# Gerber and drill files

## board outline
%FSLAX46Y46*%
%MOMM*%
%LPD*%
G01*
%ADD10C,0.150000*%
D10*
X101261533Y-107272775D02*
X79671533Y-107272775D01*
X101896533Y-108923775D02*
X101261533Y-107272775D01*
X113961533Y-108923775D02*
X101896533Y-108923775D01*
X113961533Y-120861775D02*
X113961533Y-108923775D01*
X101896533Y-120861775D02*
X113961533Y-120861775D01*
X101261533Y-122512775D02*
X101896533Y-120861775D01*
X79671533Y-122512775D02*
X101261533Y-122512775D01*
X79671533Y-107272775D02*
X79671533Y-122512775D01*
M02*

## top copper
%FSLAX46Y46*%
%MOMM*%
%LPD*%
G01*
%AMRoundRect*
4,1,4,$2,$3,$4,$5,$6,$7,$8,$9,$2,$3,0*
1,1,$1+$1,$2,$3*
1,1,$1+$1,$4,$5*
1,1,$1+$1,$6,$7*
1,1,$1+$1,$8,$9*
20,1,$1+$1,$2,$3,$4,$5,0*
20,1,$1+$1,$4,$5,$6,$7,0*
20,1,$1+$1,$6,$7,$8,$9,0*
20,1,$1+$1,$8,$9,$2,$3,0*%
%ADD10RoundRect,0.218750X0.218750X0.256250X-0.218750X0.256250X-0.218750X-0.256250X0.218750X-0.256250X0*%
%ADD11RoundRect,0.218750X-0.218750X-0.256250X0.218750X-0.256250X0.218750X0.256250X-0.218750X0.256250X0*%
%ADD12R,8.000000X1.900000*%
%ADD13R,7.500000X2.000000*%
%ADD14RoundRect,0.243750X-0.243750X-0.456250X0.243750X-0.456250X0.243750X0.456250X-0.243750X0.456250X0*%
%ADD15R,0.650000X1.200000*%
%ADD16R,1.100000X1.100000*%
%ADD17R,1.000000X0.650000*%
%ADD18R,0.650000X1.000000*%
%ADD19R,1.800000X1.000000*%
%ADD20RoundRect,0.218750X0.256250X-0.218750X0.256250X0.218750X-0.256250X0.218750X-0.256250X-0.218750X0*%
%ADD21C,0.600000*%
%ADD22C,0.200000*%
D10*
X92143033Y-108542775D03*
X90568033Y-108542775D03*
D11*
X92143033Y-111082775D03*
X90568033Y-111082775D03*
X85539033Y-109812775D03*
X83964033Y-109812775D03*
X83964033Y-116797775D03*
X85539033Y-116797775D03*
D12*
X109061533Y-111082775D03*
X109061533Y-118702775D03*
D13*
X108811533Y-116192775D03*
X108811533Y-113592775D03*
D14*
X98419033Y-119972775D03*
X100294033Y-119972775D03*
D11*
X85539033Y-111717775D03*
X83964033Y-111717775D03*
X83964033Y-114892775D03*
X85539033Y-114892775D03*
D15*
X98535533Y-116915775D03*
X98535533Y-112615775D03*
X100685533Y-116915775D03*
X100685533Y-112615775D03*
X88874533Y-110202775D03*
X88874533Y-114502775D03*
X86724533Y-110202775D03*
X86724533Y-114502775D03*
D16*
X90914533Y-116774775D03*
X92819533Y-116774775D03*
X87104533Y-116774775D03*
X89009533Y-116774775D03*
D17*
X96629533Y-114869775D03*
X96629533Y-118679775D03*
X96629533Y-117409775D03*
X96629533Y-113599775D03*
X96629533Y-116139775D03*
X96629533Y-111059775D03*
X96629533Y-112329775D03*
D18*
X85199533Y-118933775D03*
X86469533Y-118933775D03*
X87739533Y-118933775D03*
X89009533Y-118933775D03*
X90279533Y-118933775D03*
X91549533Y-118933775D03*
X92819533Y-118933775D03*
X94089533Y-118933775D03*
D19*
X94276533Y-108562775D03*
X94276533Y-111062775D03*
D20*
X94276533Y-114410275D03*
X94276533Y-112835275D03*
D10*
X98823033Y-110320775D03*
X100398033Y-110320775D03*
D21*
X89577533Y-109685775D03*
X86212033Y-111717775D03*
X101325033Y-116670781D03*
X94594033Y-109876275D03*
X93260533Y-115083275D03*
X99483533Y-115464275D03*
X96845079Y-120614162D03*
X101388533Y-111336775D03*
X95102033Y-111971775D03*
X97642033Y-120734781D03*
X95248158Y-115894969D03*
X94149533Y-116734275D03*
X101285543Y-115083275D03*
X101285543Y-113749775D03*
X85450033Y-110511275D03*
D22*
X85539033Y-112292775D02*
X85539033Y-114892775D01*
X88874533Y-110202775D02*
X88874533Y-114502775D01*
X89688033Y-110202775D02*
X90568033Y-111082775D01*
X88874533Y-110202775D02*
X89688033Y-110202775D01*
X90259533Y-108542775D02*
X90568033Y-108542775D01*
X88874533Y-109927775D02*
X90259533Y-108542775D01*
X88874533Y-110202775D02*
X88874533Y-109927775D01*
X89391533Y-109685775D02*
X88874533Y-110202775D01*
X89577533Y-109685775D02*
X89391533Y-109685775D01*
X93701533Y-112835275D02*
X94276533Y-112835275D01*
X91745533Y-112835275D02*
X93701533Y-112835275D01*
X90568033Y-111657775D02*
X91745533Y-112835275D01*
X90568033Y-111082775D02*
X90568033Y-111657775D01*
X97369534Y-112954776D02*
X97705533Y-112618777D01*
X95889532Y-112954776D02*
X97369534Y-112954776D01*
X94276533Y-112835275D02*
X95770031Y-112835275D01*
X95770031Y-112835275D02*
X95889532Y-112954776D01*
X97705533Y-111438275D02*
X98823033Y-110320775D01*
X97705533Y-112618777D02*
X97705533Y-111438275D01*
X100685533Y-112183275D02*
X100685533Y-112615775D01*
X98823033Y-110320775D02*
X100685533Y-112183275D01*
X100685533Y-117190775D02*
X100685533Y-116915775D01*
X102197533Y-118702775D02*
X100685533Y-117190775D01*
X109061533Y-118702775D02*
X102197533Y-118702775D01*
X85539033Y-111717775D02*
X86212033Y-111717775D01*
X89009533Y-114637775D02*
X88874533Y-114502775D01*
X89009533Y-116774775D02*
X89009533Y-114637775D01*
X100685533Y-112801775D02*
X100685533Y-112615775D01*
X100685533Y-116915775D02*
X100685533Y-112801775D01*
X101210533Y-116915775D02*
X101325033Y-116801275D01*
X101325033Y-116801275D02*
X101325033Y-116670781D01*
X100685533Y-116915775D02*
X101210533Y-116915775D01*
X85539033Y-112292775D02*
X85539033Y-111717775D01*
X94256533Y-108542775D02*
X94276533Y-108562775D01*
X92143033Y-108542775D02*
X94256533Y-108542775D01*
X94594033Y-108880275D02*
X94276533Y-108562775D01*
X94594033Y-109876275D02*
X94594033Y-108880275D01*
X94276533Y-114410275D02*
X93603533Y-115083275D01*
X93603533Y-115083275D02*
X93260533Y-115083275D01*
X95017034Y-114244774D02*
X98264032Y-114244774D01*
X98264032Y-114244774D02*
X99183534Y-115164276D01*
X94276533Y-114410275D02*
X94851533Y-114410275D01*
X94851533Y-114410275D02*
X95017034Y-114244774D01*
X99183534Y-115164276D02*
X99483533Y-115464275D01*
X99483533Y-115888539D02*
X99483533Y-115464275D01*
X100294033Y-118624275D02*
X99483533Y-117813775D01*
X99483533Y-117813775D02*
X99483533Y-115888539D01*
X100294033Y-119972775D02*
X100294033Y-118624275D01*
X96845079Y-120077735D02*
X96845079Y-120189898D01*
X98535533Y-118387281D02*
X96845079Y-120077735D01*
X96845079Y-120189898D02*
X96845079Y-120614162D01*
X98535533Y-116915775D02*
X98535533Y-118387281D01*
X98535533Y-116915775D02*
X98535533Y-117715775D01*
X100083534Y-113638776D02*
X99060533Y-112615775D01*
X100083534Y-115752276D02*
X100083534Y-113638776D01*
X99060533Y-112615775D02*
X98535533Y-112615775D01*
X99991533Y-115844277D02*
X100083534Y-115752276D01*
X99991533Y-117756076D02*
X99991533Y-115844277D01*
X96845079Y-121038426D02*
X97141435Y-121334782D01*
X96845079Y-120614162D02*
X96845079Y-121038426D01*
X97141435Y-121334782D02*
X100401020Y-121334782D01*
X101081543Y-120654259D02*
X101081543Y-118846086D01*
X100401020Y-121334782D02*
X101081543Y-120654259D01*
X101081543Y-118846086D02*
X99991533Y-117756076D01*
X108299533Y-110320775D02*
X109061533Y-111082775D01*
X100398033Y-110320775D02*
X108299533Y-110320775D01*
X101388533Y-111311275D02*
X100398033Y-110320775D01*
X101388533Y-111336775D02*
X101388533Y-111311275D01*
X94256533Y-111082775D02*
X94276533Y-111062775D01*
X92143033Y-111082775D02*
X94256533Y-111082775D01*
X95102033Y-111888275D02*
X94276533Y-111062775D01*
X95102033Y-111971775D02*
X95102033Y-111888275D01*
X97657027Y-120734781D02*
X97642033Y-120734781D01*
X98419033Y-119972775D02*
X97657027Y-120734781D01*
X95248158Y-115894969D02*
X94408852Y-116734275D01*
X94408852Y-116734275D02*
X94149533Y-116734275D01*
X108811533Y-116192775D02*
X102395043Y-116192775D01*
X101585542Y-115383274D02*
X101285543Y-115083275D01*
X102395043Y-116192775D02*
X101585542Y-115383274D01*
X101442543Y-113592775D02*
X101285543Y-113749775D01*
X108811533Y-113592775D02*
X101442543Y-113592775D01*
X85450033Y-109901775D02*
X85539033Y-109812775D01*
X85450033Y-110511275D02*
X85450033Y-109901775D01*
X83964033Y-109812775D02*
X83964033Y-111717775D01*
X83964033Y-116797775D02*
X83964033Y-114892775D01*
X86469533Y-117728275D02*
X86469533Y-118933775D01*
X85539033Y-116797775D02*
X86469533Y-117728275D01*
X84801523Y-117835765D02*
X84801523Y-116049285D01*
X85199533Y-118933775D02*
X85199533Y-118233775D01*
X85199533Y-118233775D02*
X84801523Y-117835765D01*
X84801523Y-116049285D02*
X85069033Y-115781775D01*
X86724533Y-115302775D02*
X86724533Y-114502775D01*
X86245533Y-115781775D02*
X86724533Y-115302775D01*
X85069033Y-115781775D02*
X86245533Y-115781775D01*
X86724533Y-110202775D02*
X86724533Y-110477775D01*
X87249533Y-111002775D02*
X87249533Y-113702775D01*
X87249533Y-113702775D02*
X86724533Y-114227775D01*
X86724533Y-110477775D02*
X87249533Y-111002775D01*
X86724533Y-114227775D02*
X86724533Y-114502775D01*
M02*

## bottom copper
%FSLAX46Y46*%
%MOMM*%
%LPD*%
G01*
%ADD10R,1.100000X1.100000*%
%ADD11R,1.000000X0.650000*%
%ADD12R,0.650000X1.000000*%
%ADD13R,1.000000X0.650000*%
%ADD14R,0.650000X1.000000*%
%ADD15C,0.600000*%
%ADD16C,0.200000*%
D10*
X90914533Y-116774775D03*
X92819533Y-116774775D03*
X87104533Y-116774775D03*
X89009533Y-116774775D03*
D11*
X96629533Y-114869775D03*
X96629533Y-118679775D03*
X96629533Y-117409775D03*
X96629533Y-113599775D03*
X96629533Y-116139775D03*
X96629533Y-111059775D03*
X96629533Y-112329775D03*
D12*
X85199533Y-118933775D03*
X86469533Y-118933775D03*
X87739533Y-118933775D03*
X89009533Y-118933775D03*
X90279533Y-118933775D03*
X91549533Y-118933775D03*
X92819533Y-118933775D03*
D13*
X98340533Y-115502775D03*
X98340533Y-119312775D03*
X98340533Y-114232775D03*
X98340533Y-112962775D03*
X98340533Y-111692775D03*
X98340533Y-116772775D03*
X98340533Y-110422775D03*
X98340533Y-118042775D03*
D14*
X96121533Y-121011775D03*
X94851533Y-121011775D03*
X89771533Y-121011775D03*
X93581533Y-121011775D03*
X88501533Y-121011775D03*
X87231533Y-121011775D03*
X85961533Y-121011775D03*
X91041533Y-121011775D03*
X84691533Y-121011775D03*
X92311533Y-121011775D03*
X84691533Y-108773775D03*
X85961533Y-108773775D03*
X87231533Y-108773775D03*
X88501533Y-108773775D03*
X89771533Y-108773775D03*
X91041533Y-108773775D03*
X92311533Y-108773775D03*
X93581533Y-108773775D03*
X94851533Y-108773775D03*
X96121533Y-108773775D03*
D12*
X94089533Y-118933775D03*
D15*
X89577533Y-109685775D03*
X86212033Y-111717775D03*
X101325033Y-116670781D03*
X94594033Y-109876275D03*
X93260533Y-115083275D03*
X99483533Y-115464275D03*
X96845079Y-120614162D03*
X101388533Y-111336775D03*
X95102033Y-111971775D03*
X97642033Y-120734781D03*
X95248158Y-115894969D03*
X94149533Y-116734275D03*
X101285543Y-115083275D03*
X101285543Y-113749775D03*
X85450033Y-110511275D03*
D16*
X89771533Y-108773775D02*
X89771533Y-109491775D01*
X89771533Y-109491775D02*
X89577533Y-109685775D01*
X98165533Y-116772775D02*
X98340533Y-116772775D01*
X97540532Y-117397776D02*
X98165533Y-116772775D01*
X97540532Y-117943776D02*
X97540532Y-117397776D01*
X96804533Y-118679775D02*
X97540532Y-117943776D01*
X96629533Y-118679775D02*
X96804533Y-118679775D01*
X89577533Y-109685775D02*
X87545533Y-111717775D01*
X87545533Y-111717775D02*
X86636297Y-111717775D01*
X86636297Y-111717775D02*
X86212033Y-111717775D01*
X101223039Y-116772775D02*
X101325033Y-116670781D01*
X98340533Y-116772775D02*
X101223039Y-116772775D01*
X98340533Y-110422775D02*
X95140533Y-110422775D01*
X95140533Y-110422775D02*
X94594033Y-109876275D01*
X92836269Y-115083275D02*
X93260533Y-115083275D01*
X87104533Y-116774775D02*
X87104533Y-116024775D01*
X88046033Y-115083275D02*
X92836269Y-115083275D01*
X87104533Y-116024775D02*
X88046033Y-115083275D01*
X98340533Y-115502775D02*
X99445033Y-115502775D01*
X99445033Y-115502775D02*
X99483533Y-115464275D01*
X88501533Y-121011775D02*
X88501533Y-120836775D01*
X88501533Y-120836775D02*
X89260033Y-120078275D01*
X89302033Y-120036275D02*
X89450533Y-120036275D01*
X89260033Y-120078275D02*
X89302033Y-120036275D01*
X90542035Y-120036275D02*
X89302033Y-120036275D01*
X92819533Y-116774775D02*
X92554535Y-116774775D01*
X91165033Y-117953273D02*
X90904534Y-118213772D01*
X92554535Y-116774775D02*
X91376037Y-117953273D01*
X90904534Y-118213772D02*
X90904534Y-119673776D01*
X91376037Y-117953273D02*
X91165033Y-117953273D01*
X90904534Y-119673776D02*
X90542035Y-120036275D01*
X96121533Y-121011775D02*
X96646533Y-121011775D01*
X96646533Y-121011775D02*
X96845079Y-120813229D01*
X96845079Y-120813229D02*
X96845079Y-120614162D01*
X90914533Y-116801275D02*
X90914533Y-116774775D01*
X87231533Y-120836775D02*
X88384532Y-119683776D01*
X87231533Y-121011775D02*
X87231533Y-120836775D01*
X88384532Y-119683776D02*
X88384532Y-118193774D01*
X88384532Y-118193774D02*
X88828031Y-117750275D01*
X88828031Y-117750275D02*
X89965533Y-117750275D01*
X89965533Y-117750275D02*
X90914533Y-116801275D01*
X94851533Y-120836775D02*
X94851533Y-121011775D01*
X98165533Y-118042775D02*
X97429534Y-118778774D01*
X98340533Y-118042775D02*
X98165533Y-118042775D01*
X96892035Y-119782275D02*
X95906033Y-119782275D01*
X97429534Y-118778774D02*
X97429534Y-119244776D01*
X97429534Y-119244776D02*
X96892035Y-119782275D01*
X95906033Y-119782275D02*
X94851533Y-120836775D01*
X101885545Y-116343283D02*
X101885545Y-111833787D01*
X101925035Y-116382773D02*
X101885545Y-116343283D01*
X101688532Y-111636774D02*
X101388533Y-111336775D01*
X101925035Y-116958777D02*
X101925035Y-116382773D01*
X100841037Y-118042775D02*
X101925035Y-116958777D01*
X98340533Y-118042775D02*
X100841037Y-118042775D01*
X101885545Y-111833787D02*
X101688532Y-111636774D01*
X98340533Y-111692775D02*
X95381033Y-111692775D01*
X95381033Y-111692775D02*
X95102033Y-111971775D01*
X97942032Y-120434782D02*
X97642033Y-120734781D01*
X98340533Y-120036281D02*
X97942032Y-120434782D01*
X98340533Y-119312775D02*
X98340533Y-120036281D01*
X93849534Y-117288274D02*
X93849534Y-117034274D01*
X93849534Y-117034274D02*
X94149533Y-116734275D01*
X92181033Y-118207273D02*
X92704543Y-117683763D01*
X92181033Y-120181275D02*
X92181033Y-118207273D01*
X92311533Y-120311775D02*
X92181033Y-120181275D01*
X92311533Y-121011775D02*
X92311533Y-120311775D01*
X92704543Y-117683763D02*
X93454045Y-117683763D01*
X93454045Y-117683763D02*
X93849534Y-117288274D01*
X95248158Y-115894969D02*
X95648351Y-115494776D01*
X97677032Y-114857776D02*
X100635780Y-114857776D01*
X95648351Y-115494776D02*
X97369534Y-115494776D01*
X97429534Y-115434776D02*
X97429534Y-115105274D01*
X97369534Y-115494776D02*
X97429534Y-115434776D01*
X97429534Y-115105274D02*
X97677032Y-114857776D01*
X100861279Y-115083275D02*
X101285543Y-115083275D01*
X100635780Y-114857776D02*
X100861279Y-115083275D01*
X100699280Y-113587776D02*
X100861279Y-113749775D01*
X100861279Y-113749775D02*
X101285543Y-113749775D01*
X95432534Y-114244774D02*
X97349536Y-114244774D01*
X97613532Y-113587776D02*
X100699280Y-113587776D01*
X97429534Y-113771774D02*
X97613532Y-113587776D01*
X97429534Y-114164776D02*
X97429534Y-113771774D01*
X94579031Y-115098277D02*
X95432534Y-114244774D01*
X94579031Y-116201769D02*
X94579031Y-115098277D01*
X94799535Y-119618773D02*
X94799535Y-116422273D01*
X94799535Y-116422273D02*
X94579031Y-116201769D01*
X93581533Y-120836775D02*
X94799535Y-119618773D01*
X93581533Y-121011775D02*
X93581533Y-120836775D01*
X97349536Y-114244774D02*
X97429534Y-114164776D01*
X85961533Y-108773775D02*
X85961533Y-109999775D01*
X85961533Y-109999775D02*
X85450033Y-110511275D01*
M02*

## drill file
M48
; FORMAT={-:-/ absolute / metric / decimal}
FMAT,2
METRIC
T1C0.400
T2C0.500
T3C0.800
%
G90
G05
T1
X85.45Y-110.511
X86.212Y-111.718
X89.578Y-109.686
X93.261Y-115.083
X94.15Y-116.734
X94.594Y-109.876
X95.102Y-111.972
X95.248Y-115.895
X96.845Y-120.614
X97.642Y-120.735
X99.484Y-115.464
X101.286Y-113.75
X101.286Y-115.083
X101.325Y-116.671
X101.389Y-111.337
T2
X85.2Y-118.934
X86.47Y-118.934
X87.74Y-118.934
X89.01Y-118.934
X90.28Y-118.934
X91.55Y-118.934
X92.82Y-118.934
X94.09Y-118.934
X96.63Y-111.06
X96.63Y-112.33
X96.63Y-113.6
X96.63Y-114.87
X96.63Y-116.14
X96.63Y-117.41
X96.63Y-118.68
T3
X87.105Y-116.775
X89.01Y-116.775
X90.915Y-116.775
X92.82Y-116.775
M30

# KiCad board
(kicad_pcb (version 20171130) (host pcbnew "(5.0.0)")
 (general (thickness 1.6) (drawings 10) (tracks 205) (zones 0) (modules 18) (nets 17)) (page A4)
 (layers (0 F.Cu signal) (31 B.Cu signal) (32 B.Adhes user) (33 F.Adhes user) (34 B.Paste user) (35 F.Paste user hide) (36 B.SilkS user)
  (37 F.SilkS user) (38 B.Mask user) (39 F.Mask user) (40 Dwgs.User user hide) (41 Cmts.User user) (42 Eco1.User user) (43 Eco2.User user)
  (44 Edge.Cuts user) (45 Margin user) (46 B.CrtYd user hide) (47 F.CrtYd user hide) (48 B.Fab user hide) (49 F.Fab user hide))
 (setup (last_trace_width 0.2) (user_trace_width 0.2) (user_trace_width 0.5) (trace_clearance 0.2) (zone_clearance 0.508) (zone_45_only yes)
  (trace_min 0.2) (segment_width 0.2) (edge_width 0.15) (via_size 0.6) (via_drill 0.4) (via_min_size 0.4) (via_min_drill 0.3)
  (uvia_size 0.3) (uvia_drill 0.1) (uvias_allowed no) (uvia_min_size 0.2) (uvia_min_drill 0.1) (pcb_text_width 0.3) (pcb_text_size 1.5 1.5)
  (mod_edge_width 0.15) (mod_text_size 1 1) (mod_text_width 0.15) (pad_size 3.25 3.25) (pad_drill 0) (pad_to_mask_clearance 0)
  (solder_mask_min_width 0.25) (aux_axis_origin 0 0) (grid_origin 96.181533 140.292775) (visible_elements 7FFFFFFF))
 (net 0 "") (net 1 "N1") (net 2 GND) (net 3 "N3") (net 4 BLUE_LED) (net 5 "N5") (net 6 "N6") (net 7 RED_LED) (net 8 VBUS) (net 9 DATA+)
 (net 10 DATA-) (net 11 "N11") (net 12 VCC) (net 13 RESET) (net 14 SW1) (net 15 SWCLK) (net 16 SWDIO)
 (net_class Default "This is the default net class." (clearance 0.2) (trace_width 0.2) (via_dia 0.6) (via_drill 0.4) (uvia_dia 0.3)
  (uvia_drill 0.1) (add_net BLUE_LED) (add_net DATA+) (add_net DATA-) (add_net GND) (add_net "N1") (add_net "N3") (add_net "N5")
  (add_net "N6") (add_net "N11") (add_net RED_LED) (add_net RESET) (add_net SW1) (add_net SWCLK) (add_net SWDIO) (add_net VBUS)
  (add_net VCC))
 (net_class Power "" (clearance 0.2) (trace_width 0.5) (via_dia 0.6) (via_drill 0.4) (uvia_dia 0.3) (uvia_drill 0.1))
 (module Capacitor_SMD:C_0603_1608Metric (layer F.Cu) (at 91.355533 108.542775 180)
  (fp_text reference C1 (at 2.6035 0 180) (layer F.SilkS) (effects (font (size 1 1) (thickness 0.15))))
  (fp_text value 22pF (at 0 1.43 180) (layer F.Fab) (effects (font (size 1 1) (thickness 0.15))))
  (pad 1 smd roundrect (at -0.7875 0 180) (size 0.875 0.95) (layers F.Cu F.Paste F.Mask) (roundrect_rratio 0.25) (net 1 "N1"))
  (pad 2 smd roundrect (at 0.7875 0 180) (size 0.875 0.95) (layers F.Cu F.Paste F.Mask) (roundrect_rratio 0.25) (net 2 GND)))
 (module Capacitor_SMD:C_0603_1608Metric (layer F.Cu) (at 91.355533 111.082775)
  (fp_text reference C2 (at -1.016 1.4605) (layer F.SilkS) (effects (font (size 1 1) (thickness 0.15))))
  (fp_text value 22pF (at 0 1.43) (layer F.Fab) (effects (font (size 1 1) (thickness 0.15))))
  (pad 2 smd roundrect (at 0.7875 0) (size 0.875 0.95) (layers F.Cu F.Paste F.Mask) (roundrect_rratio 0.25) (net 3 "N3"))
  (pad 1 smd roundrect (at -0.7875 0) (size 0.875 0.95) (layers F.Cu F.Paste F.Mask) (roundrect_rratio 0.25) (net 2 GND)))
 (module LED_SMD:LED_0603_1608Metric (layer F.Cu) (at 84.751533 109.812775)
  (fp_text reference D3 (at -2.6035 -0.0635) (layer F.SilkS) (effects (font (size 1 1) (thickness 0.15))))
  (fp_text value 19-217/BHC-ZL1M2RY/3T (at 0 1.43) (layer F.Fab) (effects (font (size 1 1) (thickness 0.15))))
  (pad 2 smd roundrect (at 0.7875 0) (size 0.875 0.95) (layers F.Cu F.Paste F.Mask) (roundrect_rratio 0.25) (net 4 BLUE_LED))
  (pad 1 smd roundrect (at -0.7875 0) (size 0.875 0.95) (layers F.Cu F.Paste F.Mask) (roundrect_rratio 0.25) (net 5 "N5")))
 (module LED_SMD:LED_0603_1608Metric (layer F.Cu) (at 84.751533 116.797775)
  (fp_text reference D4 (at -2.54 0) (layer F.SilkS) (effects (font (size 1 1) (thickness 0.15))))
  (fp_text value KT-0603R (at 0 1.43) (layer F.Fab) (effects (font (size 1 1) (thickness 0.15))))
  (pad 1 smd roundrect (at -0.7875 0) (size 0.875 0.95) (layers F.Cu F.Paste F.Mask) (roundrect_rratio 0.25) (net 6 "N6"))
  (pad 2 smd roundrect (at 0.7875 0) (size 0.875 0.95) (layers F.Cu F.Paste F.Mask) (roundrect_rratio 0.25) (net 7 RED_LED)))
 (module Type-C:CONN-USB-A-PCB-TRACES (layer F.Cu) (at 113.961533 114.892775 90)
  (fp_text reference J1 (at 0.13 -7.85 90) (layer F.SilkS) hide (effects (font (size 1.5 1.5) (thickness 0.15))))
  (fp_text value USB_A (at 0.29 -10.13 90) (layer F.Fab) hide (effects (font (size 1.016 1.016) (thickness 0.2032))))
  (pad 1 connect rect (at 3.81 -4.9 90) (size 1.9 8) (layers F.Cu F.Mask) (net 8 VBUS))
  (pad 4 connect rect (at -3.81 -4.9 90) (size 1.9 8) (layers F.Cu F.Mask) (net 2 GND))
  (pad 3 connect rect (at -1.3 -5.15 90) (size 2 7.5) (layers F.Cu F.Mask) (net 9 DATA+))
  (pad 2 connect rect (at 1.3 -5.15 90) (size 2 7.5) (layers F.Cu F.Mask) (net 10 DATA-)))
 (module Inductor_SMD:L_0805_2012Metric (layer F.Cu) (at 99.356533 119.972775)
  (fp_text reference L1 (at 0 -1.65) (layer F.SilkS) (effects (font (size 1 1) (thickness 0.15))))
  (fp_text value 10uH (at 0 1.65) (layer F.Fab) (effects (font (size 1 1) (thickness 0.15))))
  (pad 1 smd roundrect (at -0.9375 0) (size 0.975 1.4) (layers F.Cu F.Paste F.Mask) (roundrect_rratio 0.25) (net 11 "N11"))
  (pad 2 smd roundrect (at 0.9375 0) (size 0.975 1.4) (layers F.Cu F.Paste F.Mask) (roundrect_rratio 0.25) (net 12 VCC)))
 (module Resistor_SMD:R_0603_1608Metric (layer F.Cu) (at 84.751533 111.717775)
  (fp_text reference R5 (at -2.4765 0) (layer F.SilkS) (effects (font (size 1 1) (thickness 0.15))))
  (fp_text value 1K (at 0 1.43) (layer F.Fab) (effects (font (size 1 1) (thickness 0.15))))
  (pad 2 smd roundrect (at 0.7875 0) (size 0.875 0.95) (layers F.Cu F.Paste F.Mask) (roundrect_rratio 0.25) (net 2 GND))
  (pad 1 smd roundrect (at -0.7875 0) (size 0.875 0.95) (layers F.Cu F.Paste F.Mask) (roundrect_rratio 0.25) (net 5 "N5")))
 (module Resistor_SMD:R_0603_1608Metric (layer F.Cu) (at 84.751533 114.892775)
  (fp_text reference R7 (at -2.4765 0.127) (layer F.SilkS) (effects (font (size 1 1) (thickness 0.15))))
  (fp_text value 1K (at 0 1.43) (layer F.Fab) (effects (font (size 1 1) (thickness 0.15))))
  (pad 1 smd roundrect (at -0.7875 0) (size 0.875 0.95) (layers F.Cu F.Paste F.Mask) (roundrect_rratio 0.25) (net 6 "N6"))
  (pad 2 smd roundrect (at 0.7875 0) (size 0.875 0.95) (layers F.Cu F.Paste F.Mask) (roundrect_rratio 0.25) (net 2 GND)))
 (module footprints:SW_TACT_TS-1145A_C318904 (layer F.Cu) (at 99.610533 114.765775 270)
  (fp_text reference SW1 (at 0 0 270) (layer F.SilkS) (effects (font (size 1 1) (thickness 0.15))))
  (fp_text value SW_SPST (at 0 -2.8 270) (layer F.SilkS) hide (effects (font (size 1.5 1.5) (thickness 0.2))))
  (pad 2 smd rect (at 2.15 1.075 270) (size 1.2 0.65) (layers F.Cu F.Paste F.Mask) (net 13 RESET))
  (pad 2 smd rect (at -2.15 1.075 270) (size 1.2 0.65) (layers F.Cu F.Paste F.Mask) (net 13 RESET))
  (pad 1 smd rect (at 2.15 -1.075 270) (size 1.2 0.65) (layers F.Cu F.Paste F.Mask) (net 2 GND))
  (pad 1 smd rect (at -2.15 -1.075 270) (size 1.2 0.65) (layers F.Cu F.Paste F.Mask) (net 2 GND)))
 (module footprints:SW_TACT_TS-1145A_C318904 (layer F.Cu) (at 87.799533 112.352775 270)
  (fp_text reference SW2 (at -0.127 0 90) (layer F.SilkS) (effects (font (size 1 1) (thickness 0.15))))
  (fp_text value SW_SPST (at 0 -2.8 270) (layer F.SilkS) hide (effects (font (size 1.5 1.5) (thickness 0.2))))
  (pad 1 smd rect (at -2.15 -1.075 270) (size 1.2 0.65) (layers F.Cu F.Paste F.Mask) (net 2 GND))
  (pad 1 smd rect (at 2.15 -1.075 270) (size 1.2 0.65) (layers F.Cu F.Paste F.Mask) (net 2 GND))
  (pad 2 smd rect (at -2.15 1.075 270) (size 1.2 0.65) (layers F.Cu F.Paste F.Mask) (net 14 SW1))
  (pad 2 smd rect (at 2.15 1.075 270) (size 1.2 0.65) (layers F.Cu F.Paste F.Mask) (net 14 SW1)))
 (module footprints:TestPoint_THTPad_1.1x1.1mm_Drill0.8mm (layer F.Cu) (at 90.914533 116.774775)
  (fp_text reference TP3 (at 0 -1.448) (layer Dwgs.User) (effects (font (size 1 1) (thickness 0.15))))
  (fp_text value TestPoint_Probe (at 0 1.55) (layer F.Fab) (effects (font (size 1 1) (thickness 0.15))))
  (pad 1 thru_hole rect (at 0 0) (size 1.1 1.1) (drill 0.8) (layers *.Cu *.Mask) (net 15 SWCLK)))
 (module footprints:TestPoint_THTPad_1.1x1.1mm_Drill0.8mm (layer F.Cu) (at 92.819533 116.774775)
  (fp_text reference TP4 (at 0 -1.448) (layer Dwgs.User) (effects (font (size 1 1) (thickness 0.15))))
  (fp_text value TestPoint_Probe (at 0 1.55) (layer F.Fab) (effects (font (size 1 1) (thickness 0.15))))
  (pad 1 thru_hole rect (at 0 0) (size 1.1 1.1) (drill 0.8) (layers *.Cu *.Mask) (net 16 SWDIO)))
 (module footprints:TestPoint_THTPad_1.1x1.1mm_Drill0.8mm (layer F.Cu) (at 87.104533 116.774775)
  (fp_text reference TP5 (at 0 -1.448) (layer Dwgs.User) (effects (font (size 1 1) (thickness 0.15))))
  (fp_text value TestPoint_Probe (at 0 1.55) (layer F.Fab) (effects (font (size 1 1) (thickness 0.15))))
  (pad 1 thru_hole rect (at 0 0) (size 1.1 1.1) (drill 0.8) (layers *.Cu *.Mask) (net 12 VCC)))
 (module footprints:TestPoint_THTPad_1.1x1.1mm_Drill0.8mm (layer F.Cu) (at 89.009533 116.774775)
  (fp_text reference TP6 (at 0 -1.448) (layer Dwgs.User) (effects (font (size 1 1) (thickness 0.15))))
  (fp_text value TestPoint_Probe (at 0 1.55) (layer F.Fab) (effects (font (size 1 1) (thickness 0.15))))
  (pad 1 thru_hole rect (at 0 0) (size 1.1 1.1) (drill 0.8) (layers *.Cu *.Mask) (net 2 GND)))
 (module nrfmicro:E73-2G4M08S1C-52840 (layer B.Cu) (at 98.721533 114.892775 180)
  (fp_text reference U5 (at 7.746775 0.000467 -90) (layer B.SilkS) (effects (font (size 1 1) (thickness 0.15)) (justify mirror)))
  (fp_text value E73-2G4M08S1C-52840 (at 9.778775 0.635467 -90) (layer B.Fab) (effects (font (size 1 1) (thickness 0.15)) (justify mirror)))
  (pad 18 thru_hole rect (at 2.092 0.023 90) (size 0.65 1) (drill 0.5) (layers *.Cu *.Mask))
  (pad 24 thru_hole rect (at 2.092 -3.787 90) (size 0.65 1) (drill 0.5) (layers *.Cu *.Mask) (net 2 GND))
  (pad 22 thru_hole rect (at 2.092 -2.517 90) (size 0.65 1) (drill 0.5) (layers *.Cu *.Mask))
  (pad 16 thru_hole rect (at 2.092 1.293 90) (size 0.65 1) (drill 0.5) (layers *.Cu *.Mask))
  (pad 20 thru_hole rect (at 2.092 -1.247 90) (size 0.65 1) (drill 0.5) (layers *.Cu *.Mask))
  (pad 12 thru_hole rect (at 2.092 3.833 90) (size 0.65 1) (drill 0.5) (layers *.Cu *.Mask))
  (pad 14 thru_hole rect (at 2.092 2.563 90) (size 0.65 1) (drill 0.5) (layers *.Cu *.Mask))
  (pad 42 thru_hole rect (at 13.522 -4.041 180) (size 0.65 1) (drill 0.5) (layers *.Cu *.Mask) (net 14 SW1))
  (pad 40 thru_hole rect (at 12.252 -4.041 180) (size 0.65 1) (drill 0.5) (layers *.Cu *.Mask) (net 7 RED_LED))
  (pad 38 thru_hole rect (at 10.982 -4.041 180) (size 0.65 1) (drill 0.5) (layers *.Cu *.Mask))
  (pad 36 thru_hole rect (at 9.712 -4.041 180) (size 0.65 1) (drill 0.5) (layers *.Cu *.Mask))
  (pad 34 thru_hole rect (at 8.442 -4.041 180) (size 0.65 1) (drill 0.5) (layers *.Cu *.Mask))
  (pad 32 thru_hole rect (at 7.172 -4.041 180) (size 0.65 1) (drill 0.5) (layers *.Cu *.Mask))
  (pad 30 thru_hole rect (at 5.902 -4.041 180) (size 0.65 1) (drill 0.5) (layers *.Cu *.Mask))
  (pad 19 smd rect (at 0.381 -0.61 90) (size 0.65 1) (layers B.Cu B.Paste B.Mask) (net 12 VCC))
  (pad 25 smd rect (at 0.381 -4.42 90) (size 0.65 1) (layers B.Cu B.Paste B.Mask) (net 11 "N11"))
  (pad 17 smd rect (at 0.381 0.66 90) (size 0.65 1) (layers B.Cu B.Paste B.Mask))
  (pad 15 smd rect (at 0.381 1.93 90) (size 0.65 1) (layers B.Cu B.Paste B.Mask))
  (pad 13 smd rect (at 0.381 3.2 90) (size 0.65 1) (layers B.Cu B.Paste B.Mask) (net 3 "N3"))
  (pad 21 smd rect (at 0.381 -1.88 90) (size 0.65 1) (layers B.Cu B.Paste B.Mask) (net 2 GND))
  (pad 11 smd rect (at 0.381 4.47 90) (size 0.65 1) (layers B.Cu B.Paste B.Mask) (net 1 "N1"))
  (pad 23 smd rect (at 0.381 -3.15 90) (size 0.65 1) (layers B.Cu B.Paste B.Mask) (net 8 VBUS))
  (pad 26 smd rect (at 2.6 -6.119 180) (size 0.65 1) (layers B.Cu B.Paste B.Mask) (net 13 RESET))
  (pad 27 smd rect (at 3.87 -6.119 180) (size 0.65 1) (layers B.Cu B.Paste B.Mask) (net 8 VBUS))
  (pad 35 smd rect (at 8.95 -6.119 180) (size 0.65 1) (layers B.Cu B.Paste B.Mask))
  (pad 29 smd rect (at 5.14 -6.119 180) (size 0.65 1) (layers B.Cu B.Paste B.Mask) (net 10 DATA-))
  (pad 37 smd rect (at 10.22 -6.119 180) (size 0.65 1) (layers B.Cu B.Paste B.Mask) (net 16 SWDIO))
  (pad 39 smd rect (at 11.49 -6.119 180) (size 0.65 1) (layers B.Cu B.Paste B.Mask) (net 15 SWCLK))
  (pad 41 smd rect (at 12.76 -6.119 180) (size 0.65 1) (layers B.Cu B.Paste B.Mask))
  (pad 33 smd rect (at 7.68 -6.119 180) (size 0.65 1) (layers B.Cu B.Paste B.Mask))
  (pad 43 smd rect (at 14.03 -6.119 180) (size 0.65 1) (layers B.Cu B.Paste B.Mask))
  (pad 31 smd rect (at 6.41 -6.119 180) (size 0.65 1) (layers B.Cu B.Paste B.Mask) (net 9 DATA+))
  (pad 1 smd rect (at 14.03 6.119 180) (size 0.65 1) (layers B.Cu B.Paste B.Mask))
  (pad 2 smd rect (at 12.76 6.119 180) (size 0.65 1) (layers B.Cu B.Paste B.Mask) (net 4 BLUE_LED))
  (pad 3 smd rect (at 11.49 6.119 180) (size 0.65 1) (layers B.Cu B.Paste B.Mask))
  (pad 4 smd rect (at 10.22 6.119 180) (size 0.65 1) (layers B.Cu B.Paste B.Mask))
  (pad 5 smd rect (at 8.95 6.119 180) (size 0.65 1) (layers B.Cu B.Paste B.Mask) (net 2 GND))
  (pad 6 smd rect (at 7.68 6.119 180) (size 0.65 1) (layers B.Cu B.Paste B.Mask))
  (pad 7 smd rect (at 6.41 6.119 180) (size 0.65 1) (layers B.Cu B.Paste B.Mask))
  (pad 8 smd rect (at 5.14 6.119 180) (size 0.65 1) (layers B.Cu B.Paste B.Mask))
  (pad 9 smd rect (at 3.87 6.119 180) (size 0.65 1) (layers B.Cu B.Paste B.Mask))
  (pad 10 smd rect (at 2.6 6.119 180) (size 0.65 1) (layers B.Cu B.Paste B.Mask))
  (pad 28 thru_hole rect (at 4.632 -4.041 180) (size 0.65 1) (drill 0.5) (layers *.Cu *.Mask)))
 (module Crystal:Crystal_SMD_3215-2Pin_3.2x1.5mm (layer F.Cu) (at 94.276533 109.812775 90)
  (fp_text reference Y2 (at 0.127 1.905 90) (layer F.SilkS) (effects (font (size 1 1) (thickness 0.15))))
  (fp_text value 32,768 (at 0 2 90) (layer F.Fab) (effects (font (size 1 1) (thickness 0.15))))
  (pad 1 smd rect (at 1.25 0 90) (size 1 1.8) (layers F.Cu F.Paste F.Mask) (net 1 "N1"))
  (pad 2 smd rect (at -1.25 0 90) (size 1 1.8) (layers F.Cu F.Paste F.Mask) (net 3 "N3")))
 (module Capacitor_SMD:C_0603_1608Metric (layer F.Cu) (at 94.276533 113.622775 90)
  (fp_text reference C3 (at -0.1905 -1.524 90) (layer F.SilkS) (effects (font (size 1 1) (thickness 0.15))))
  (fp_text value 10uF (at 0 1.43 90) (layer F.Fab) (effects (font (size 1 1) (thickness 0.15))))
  (pad 1 smd roundrect (at -0.7875 0 90) (size 0.875 0.95) (layers F.Cu F.Paste F.Mask) (roundrect_rratio 0.25) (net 12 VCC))
  (pad 2 smd roundrect (at 0.7875 0 90) (size 0.875 0.95) (layers F.Cu F.Paste F.Mask) (roundrect_rratio 0.25) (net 2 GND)))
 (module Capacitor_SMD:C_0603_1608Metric (layer F.Cu) (at 99.610533 110.320775 180)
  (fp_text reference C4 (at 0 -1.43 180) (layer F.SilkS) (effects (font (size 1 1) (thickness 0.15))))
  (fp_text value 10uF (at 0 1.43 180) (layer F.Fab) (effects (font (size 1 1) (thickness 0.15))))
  (pad 2 smd roundrect (at 0.7875 0 180) (size 0.875 0.95) (layers F.Cu F.Paste F.Mask) (roundrect_rratio 0.25) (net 2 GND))
  (pad 1 smd roundrect (at -0.7875 0 180) (size 0.875 0.95) (layers F.Cu F.Paste F.Mask) (roundrect_rratio 0.25) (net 8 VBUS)))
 (gr_line (start 101.261533 107.272775) (end 79.671533 107.272775) (layer Edge.Cuts) (width 0.15))
 (gr_line (start 101.896533 108.923775) (end 101.261533 107.272775) (layer Edge.Cuts) (width 0.15))
 (gr_line (start 113.961533 108.923775) (end 101.896533 108.923775) (layer Edge.Cuts) (width 0.15))
 (gr_line (start 113.961533 120.861775) (end 113.961533 108.923775) (layer Edge.Cuts) (width 0.15))
 (gr_line (start 101.896533 120.861775) (end 113.961533 120.861775) (layer Edge.Cuts) (width 0.15))
 (gr_line (start 101.261533 122.512775) (end 101.896533 120.861775) (layer Edge.Cuts) (width 0.15))
 (gr_line (start 79.671533 122.512775) (end 101.261533 122.512775) (layer Edge.Cuts) (width 0.15))
 (gr_line (start 79.671533 107.272775) (end 79.671533 122.512775) (layer Edge.Cuts) (width 0.15))
 (segment (start 85.539033 112.292775) (end 85.539033 114.892775) (width 0.2) (layer F.Cu) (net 2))
 (segment (start 88.874533 110.202775) (end 88.874533 114.502775) (width 0.2) (layer F.Cu) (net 2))
 (segment (start 89.688033 110.202775) (end 90.568033 111.082775) (width 0.2) (layer F.Cu) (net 2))
 (segment (start 88.874533 110.202775) (end 89.688033 110.202775) (width 0.2) (layer F.Cu) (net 2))
 (segment (start 90.259533 108.542775) (end 90.568033 108.542775) (width 0.2) (layer F.Cu) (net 2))
 (segment (start 88.874533 109.927775) (end 90.259533 108.542775) (width 0.2) (layer F.Cu) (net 2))
 (segment (start 88.874533 110.202775) (end 88.874533 109.927775) (width 0.2) (layer F.Cu) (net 2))
 (via (at 89.577533 109.685775) (size 0.6) (drill 0.4) (layers F.Cu B.Cu) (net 2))
 (segment (start 89.771533 108.773775) (end 89.771533 109.491775) (width 0.2) (layer B.Cu) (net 2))
 (segment (start 89.771533 109.491775) (end 89.577533 109.685775) (width 0.2) (layer B.Cu) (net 2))
 (segment (start 89.391533 109.685775) (end 88.874533 110.202775) (width 0.2) (layer F.Cu) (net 2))
 (segment (start 89.577533 109.685775) (end 89.391533 109.685775) (width 0.2) (layer F.Cu) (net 2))
 (segment (start 93.701533 112.835275) (end 94.276533 112.835275) (width 0.2) (layer F.Cu) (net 2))
 (segment (start 91.745533 112.835275) (end 93.701533 112.835275) (width 0.2) (layer F.Cu) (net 2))
 (segment (start 90.568033 111.657775) (end 91.745533 112.835275) (width 0.2) (layer F.Cu) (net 2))
 (segment (start 90.568033 111.082775) (end 90.568033 111.657775) (width 0.2) (layer F.Cu) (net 2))
 (segment (start 97.369534 112.954776) (end 97.705533 112.618777) (width 0.2) (layer F.Cu) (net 2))
 (segment (start 95.889532 112.954776) (end 97.369534 112.954776) (width 0.2) (layer F.Cu) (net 2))
 (segment (start 94.276533 112.835275) (end 95.770031 112.835275) (width 0.2) (layer F.Cu) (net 2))
 (segment (start 95.770031 112.835275) (end 95.889532 112.954776) (width 0.2) (layer F.Cu) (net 2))
 (segment (start 97.705533 111.438275) (end 98.823033 110.320775) (width 0.2) (layer F.Cu) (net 2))
 (segment (start 97.705533 112.618777) (end 97.705533 111.438275) (width 0.2) (layer F.Cu) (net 2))
 (segment (start 100.685533 112.183275) (end 100.685533 112.615775) (width 0.2) (layer F.Cu) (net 2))
 (segment (start 98.823033 110.320775) (end 100.685533 112.183275) (width 0.2) (layer F.Cu) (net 2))
 (segment (start 100.685533 117.190775) (end 100.685533 116.915775) (width 0.2) (layer F.Cu) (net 2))
 (segment (start 102.197533 118.702775) (end 100.685533 117.190775) (width 0.2) (layer F.Cu) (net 2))
 (segment (start 109.061533 118.702775) (end 102.197533 118.702775) (width 0.2) (layer F.Cu) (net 2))
 (segment (start 98.165533 116.772775) (end 98.340533 116.772775) (width 0.2) (layer B.Cu) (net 2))
 (segment (start 97.540532 117.397776) (end 98.165533 116.772775) (width 0.2) (layer B.Cu) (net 2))
 (segment (start 97.540532 117.943776) (end 97.540532 117.397776) (width 0.2) (layer B.Cu) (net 2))
 (segment (start 96.804533 118.679775) (end 97.540532 117.943776) (width 0.2) (layer B.Cu) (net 2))
 (segment (start 96.629533 118.679775) (end 96.804533 118.679775) (width 0.2) (layer B.Cu) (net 2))
 (segment (start 85.539033 111.717775) (end 86.212033 111.717775) (width 0.2) (layer F.Cu) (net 2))
 (segment (start 89.577533 109.685775) (end 87.545533 111.717775) (width 0.2) (layer B.Cu) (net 2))
 (via (at 86.212033 111.717775) (size 0.6) (drill 0.4) (layers F.Cu B.Cu) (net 2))
 (segment (start 87.545533 111.717775) (end 86.636297 111.717775) (width 0.2) (layer B.Cu) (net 2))
 (segment (start 86.636297 111.717775) (end 86.212033 111.717775) (width 0.2) (layer B.Cu) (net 2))
 (segment (start 89.009533 114.637775) (end 88.874533 114.502775) (width 0.2) (layer F.Cu) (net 2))
 (segment (start 89.009533 116.774775) (end 89.009533 114.637775) (width 0.2) (layer F.Cu) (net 2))
 (segment (start 100.685533 112.801775) (end 100.685533 112.615775) (width 0.2) (layer F.Cu) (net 2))
 (segment (start 100.685533 116.915775) (end 100.685533 112.801775) (width 0.2) (layer F.Cu) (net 2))
 (via (at 101.325033 116.670781) (size 0.6) (drill 0.4) (layers F.Cu B.Cu) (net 2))
 (segment (start 101.210533 116.915775) (end 101.325033 116.801275) (width 0.2) (layer F.Cu) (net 2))
 (segment (start 101.325033 116.801275) (end 101.325033 116.670781) (width 0.2) (layer F.Cu) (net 2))
 (segment (start 100.685533 116.915775) (end 101.210533 116.915775) (width 0.2) (layer F.Cu) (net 2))
 (segment (start 101.223039 116.772775) (end 101.325033 116.670781) (width 0.2) (layer B.Cu) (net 2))
 (segment (start 98.340533 116.772775) (end 101.223039 116.772775) (width 0.2) (layer B.Cu) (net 2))
 (segment (start 85.539033 112.292775) (end 85.539033 111.717775) (width 0.2) (layer F.Cu) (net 2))
 (segment (start 94.256533 108.542775) (end 94.276533 108.562775) (width 0.2) (layer F.Cu) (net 1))
 (segment (start 92.143033 108.542775) (end 94.256533 108.542775) (width 0.2) (layer F.Cu) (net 1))
 (via (at 94.594033 109.876275) (size 0.6) (drill 0.4) (layers F.Cu B.Cu) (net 1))
 (segment (start 98.340533 110.422775) (end 95.140533 110.422775) (width 0.2) (layer B.Cu) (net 1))
 (segment (start 95.140533 110.422775) (end 94.594033 109.876275) (width 0.2) (layer B.Cu) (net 1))
 (segment (start 94.594033 108.880275) (end 94.276533 108.562775) (width 0.2) (layer F.Cu) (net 1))
 (segment (start 94.594033 109.876275) (end 94.594033 108.880275) (width 0.2) (layer F.Cu) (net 1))
 (segment (start 92.836269 115.083275) (end 93.260533 115.083275) (width 0.2) (layer B.Cu) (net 12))
 (segment (start 87.104533 116.774775) (end 87.104533 116.024775) (width 0.2) (layer B.Cu) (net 12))
 (segment (start 94.276533 114.410275) (end 93.603533 115.083275) (width 0.2) (layer F.Cu) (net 12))
 (segment (start 88.046033 115.083275) (end 92.836269 115.083275) (width 0.2) (layer B.Cu) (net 12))
 (segment (start 93.603533 115.083275) (end 93.260533 115.083275) (width 0.2) (layer F.Cu) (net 12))
 (segment (start 87.104533 116.024775) (end 88.046033 115.083275) (width 0.2) (layer B.Cu) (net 12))
 (via (at 93.260533 115.083275) (size 0.6) (drill 0.4) (layers F.Cu B.Cu) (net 12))
 (segment (start 95.017034 114.244774) (end 98.264032 114.244774) (width 0.2) (layer F.Cu) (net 12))
 (segment (start 98.264032 114.244774) (end 99.183534 115.164276) (width 0.2) (layer F.Cu) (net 12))
 (segment (start 98.340533 115.502775) (end 99.445033 115.502775) (width 0.2) (layer B.Cu) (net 12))
 (segment (start 94.276533 114.410275) (end 94.851533 114.410275) (width 0.2) (layer F.Cu) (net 12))
 (segment (start 94.851533 114.410275) (end 95.017034 114.244774) (width 0.2) (layer F.Cu) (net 12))
 (segment (start 99.183534 115.164276) (end 99.483533 115.464275) (width 0.2) (layer F.Cu) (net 12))
 (segment (start 99.445033 115.502775) (end 99.483533 115.464275) (width 0.2) (layer B.Cu) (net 12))
 (via (at 99.483533 115.464275) (size 0.6) (drill 0.4) (layers F.Cu B.Cu) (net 12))
 (segment (start 99.483533 115.888539) (end 99.483533 115.464275) (width 0.2) (layer F.Cu) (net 12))
 (segment (start 100.294033 118.624275) (end 99.483533 117.813775) (width 0.2) (layer F.Cu) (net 12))
 (segment (start 99.483533 117.813775) (end 99.483533 115.888539) (width 0.2) (layer F.Cu) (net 12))
 (segment (start 100.294033 119.972775) (end 100.294033 118.624275) (width 0.2) (layer F.Cu) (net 12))
 (segment (start 88.501533 121.011775) (end 88.501533 120.836775) (width 0.2) (layer B.Cu) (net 16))
 (segment (start 88.501533 120.836775) (end 89.260033 120.078275) (width 0.2) (layer B.Cu) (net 16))
 (segment (start 89.302033 120.036275) (end 89.450533 120.036275) (width 0.2) (layer B.Cu) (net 16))
 (segment (start 89.260033 120.078275) (end 89.302033 120.036275) (width 0.2) (layer B.Cu) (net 16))
 (segment (start 90.542035 120.036275) (end 89.302033 120.036275) (width 0.2) (layer B.Cu) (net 16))
 (segment (start 92.819533 116.774775) (end 92.554535 116.774775) (width 0.2) (layer B.Cu) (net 16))
 (segment (start 91.165033 117.953273) (end 90.904534 118.213772) (width 0.2) (layer B.Cu) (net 16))
 (segment (start 92.554535 116.774775) (end 91.376037 117.953273) (width 0.2) (layer B.Cu) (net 16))
 (segment (start 90.904534 118.213772) (end 90.904534 119.673776) (width 0.2) (layer B.Cu) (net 16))
 (segment (start 91.376037 117.953273) (end 91.165033 117.953273) (width 0.2) (layer B.Cu) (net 16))
 (segment (start 90.904534 119.673776) (end 90.542035 120.036275) (width 0.2) (layer B.Cu) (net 16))
 (segment (start 96.845079 120.077735) (end 96.845079 120.189898) (width 0.2) (layer F.Cu) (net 13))
 (segment (start 98.535533 118.387281) (end 96.845079 120.077735) (width 0.2) (layer F.Cu) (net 13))
 (segment (start 96.121533 121.011775) (end 96.646533 121.011775) (width 0.2) (layer B.Cu) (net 13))
 (segment (start 96.845079 120.189898) (end 96.845079 120.614162) (width 0.2) (layer F.Cu) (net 13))
 (segment (start 96.646533 121.011775) (end 96.845079 120.813229) (width 0.2) (layer B.Cu) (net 13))
 (segment (start 98.535533 116.915775) (end 98.535533 118.387281) (width 0.2) (layer F.Cu) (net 13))
 (segment (start 96.845079 120.813229) (end 96.845079 120.614162) (width 0.2) (layer B.Cu) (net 13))
 (via (at 96.845079 120.614162) (size 0.6) (drill 0.4) (layers F.Cu B.Cu) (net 13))
 (segment (start 98.535533 116.915775) (end 98.535533 117.715775) (width 0.2) (layer F.Cu) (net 13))
 (segment (start 100.083534 113.638776) (end 99.060533 112.615775) (width 0.2) (layer F.Cu) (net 13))
 (segment (start 100.083534 115.752276) (end 100.083534 113.638776) (width 0.2) (layer F.Cu) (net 13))
 (segment (start 99.060533 112.615775) (end 98.535533 112.615775) (width 0.2) (layer F.Cu) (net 13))
 (segment (start 99.991533 115.844277) (end 100.083534 115.752276) (width 0.2) (layer F.Cu) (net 13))
 (segment (start 99.991533 117.756076) (end 99.991533 115.844277) (width 0.2) (layer F.Cu) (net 13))
 (segment (start 96.845079 121.038426) (end 97.141435 121.334782) (width 0.2) (layer F.Cu) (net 13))
 (segment (start 96.845079 120.614162) (end 96.845079 121.038426) (width 0.2) (layer F.Cu) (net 13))
 (segment (start 97.141435 121.334782) (end 100.40102 121.334782) (width 0.2) (layer F.Cu) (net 13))
 (segment (start 101.081543 120.654259) (end 101.081543 118.846086) (width 0.2) (layer F.Cu) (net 13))
 (segment (start 100.40102 121.334782) (end 101.081543 120.654259) (width 0.2) (layer F.Cu) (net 13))
 (segment (start 101.081543 118.846086) (end 99.991533 117.756076) (width 0.2) (layer F.Cu) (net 13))
 (segment (start 90.914533 116.801275) (end 90.914533 116.774775) (width 0.2) (layer B.Cu) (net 15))
 (segment (start 87.231533 120.836775) (end 88.384532 119.683776) (width 0.2) (layer B.Cu) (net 15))
 (segment (start 87.231533 121.011775) (end 87.231533 120.836775) (width 0.2) (layer B.Cu) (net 15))
 (segment (start 88.384532 119.683776) (end 88.384532 118.193774) (width 0.2) (layer B.Cu) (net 15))
 (segment (start 88.384532 118.193774) (end 88.828031 117.750275) (width 0.2) (layer B.Cu) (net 15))
 (segment (start 88.828031 117.750275) (end 89.965533 117.750275) (width 0.2) (layer B.Cu) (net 15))
 (segment (start 89.965533 117.750275) (end 90.914533 116.801275) (width 0.2) (layer B.Cu) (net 15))
 (segment (start 108.299533 110.320775) (end 109.061533 111.082775) (width 0.2) (layer F.Cu) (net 8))
 (segment (start 100.398033 110.320775) (end 108.299533 110.320775) (width 0.2) (layer F.Cu) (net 8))
 (via (at 101.388533 111.336775) (size 0.6) (drill 0.4) (layers F.Cu B.Cu) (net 8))
 (segment (start 101.388533 111.311275) (end 100.398033 110.320775) (width 0.2) (layer F.Cu) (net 8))
 (segment (start 101.388533 111.336775) (end 101.388533 111.311275) (width 0.2) (layer F.Cu) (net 8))
 (segment (start 94.851533 120.836775) (end 94.851533 121.011775) (width 0.2) (layer B.Cu) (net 8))
 (segment (start 98.165533 118.042775) (end 97.429534 118.778774) (width 0.2) (layer B.Cu) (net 8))
 (segment (start 98.340533 118.042775) (end 98.165533 118.042775) (width 0.2) (layer B.Cu) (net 8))
 (segment (start 96.892035 119.782275) (end 95.906033 119.782275) (width 0.2) (layer B.Cu) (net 8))
 (segment (start 97.429534 118.778774) (end 97.429534 119.244776) (width 0.2) (layer B.Cu) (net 8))
 (segment (start 97.429534 119.244776) (end 96.892035 119.782275) (width 0.2) (layer B.Cu) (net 8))
 (segment (start 95.906033 119.782275) (end 94.851533 120.836775) (width 0.2) (layer B.Cu) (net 8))
 (segment (start 101.885545 116.343283) (end 101.885545 111.833787) (width 0.2) (layer B.Cu) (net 8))
 (segment (start 101.925035 116.382773) (end 101.885545 116.343283) (width 0.2) (layer B.Cu) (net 8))
 (segment (start 101.688532 111.636774) (end 101.388533 111.336775) (width 0.2) (layer B.Cu) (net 8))
 (segment (start 101.925035 116.958777) (end 101.925035 116.382773) (width 0.2) (layer B.Cu) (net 8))
 (segment (start 100.841037 118.042775) (end 101.925035 116.958777) (width 0.2) (layer B.Cu) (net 8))
 (segment (start 98.340533 118.042775) (end 100.841037 118.042775) (width 0.2) (layer B.Cu) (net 8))
 (segment (start 101.885545 111.833787) (end 101.688532 111.636774) (width 0.2) (layer B.Cu) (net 8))
 (segment (start 94.256533 111.082775) (end 94.276533 111.062775) (width 0.2) (layer F.Cu) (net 3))
 (segment (start 92.143033 111.082775) (end 94.256533 111.082775) (width 0.2) (layer F.Cu) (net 3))
 (via (at 95.102033 111.971775) (size 0.6) (drill 0.4) (layers F.Cu B.Cu) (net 3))
 (segment (start 98.340533 111.692775) (end 95.381033 111.692775) (width 0.2) (layer B.Cu) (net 3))
 (segment (start 95.381033 111.692775) (end 95.102033 111.971775) (width 0.2) (layer B.Cu) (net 3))
 (segment (start 95.102033 111.888275) (end 94.276533 111.062775) (width 0.2) (layer F.Cu) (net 3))
 (segment (start 95.102033 111.971775) (end 95.102033 111.888275) (width 0.2) (layer F.Cu) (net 3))
 (segment (start 97.942032 120.434782) (end 97.642033 120.734781) (width 0.2) (layer B.Cu) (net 11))
 (segment (start 97.657027 120.734781) (end 97.642033 120.734781) (width 0.2) (layer F.Cu) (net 11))
 (segment (start 98.340533 120.036281) (end 97.942032 120.434782) (width 0.2) (layer B.Cu) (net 11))
 (segment (start 98.419033 119.972775) (end 97.657027 120.734781) (width 0.2) (layer F.Cu) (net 11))
 (segment (start 98.340533 119.312775) (end 98.340533 120.036281) (width 0.2) (layer B.Cu) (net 11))
 (via (at 97.642033 120.734781) (size 0.6) (drill 0.4) (layers F.Cu B.Cu) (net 11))
 (via (at 95.248158 115.894969) (size 0.6) (drill 0.4) (layers F.Cu B.Cu) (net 9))
 (segment (start 95.248158 115.894969) (end 94.408852 116.734275) (width 0.2) (layer F.Cu) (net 9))
 (segment (start 94.408852 116.734275) (end 94.149533 116.734275) (width 0.2) (layer F.Cu) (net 9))
 (segment (start 93.849534 117.288274) (end 93.849534 117.034274) (width 0.2) (layer B.Cu) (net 9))
 (segment (start 93.849534 117.034274) (end 94.149533 116.734275) (width 0.2) (layer B.Cu) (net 9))
 (segment (start 92.181033 118.207273) (end 92.704543 117.683763) (width 0.2) (layer B.Cu) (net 9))
 (segment (start 92.181033 120.181275) (end 92.181033 118.207273) (width 0.2) (layer B.Cu) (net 9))
 (segment (start 92.311533 120.311775) (end 92.181033 120.181275) (width 0.2) (layer B.Cu) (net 9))
 (segment (start 92.311533 121.011775) (end 92.311533 120.311775) (width 0.2) (layer B.Cu) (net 9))
 (via (at 94.149533 116.734275) (size 0.6) (drill 0.4) (layers F.Cu B.Cu) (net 9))
 (segment (start 92.704543 117.683763) (end 93.454045 117.683763) (width 0.2) (layer B.Cu) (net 9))
 (segment (start 93.454045 117.683763) (end 93.849534 117.288274) (width 0.2) (layer B.Cu) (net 9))
 (segment (start 95.248158 115.894969) (end 95.648351 115.494776) (width 0.2) (layer B.Cu) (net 9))
 (segment (start 108.811533 116.192775) (end 102.395043 116.192775) (width 0.2) (layer F.Cu) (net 9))
 (via (at 101.285543 115.083275) (size 0.6) (drill 0.4) (layers F.Cu B.Cu) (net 9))
 (segment (start 97.677032 114.857776) (end 100.63578 114.857776) (width 0.2) (layer B.Cu) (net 9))
 (segment (start 101.585542 115.383274) (end 101.285543 115.083275) (width 0.2) (layer F.Cu) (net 9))
 (segment (start 95.648351 115.494776) (end 97.369534 115.494776) (width 0.2) (layer B.Cu) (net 9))
 (segment (start 97.429534 115.434776) (end 97.429534 115.105274) (width 0.2) (layer B.Cu) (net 9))
 (segment (start 97.369534 115.494776) (end 97.429534 115.434776) (width 0.2) (layer B.Cu) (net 9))
 (segment (start 97.429534 115.105274) (end 97.677032 114.857776) (width 0.2) (layer B.Cu) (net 9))
 (segment (start 100.861279 115.083275) (end 101.285543 115.083275) (width 0.2) (layer B.Cu) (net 9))
 (segment (start 100.63578 114.857776) (end 100.861279 115.083275) (width 0.2) (layer B.Cu) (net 9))
 (segment (start 102.395043 116.192775) (end 101.585542 115.383274) (width 0.2) (layer F.Cu) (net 9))
 (via (at 101.285543 113.749775) (size 0.6) (drill 0.4) (layers F.Cu B.Cu) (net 10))
 (segment (start 100.69928 113.587776) (end 100.861279 113.749775) (width 0.2) (layer B.Cu) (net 10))
 (segment (start 100.861279 113.749775) (end 101.285543 113.749775) (width 0.2) (layer B.Cu) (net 10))
 (segment (start 95.432534 114.244774) (end 97.349536 114.244774) (width 0.2) (layer B.Cu) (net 10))
 (segment (start 97.613532 113.587776) (end 100.69928 113.587776) (width 0.2) (layer B.Cu) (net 10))
 (segment (start 101.442543 113.592775) (end 101.285543 113.749775) (width 0.2) (layer F.Cu) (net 10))
 (segment (start 97.429534 113.771774) (end 97.613532 113.587776) (width 0.2) (layer B.Cu) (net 10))
 (segment (start 97.429534 114.164776) (end 97.429534 113.771774) (width 0.2) (layer B.Cu) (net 10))
 (segment (start 94.579031 115.098277) (end 95.432534 114.244774) (width 0.2) (layer B.Cu) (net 10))
 (segment (start 94.579031 116.201769) (end 94.579031 115.098277) (width 0.2) (layer B.Cu) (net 10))
 (segment (start 94.799535 119.618773) (end 94.799535 116.422273) (width 0.2) (layer B.Cu) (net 10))
 (segment (start 94.799535 116.422273) (end 94.579031 116.201769) (width 0.2) (layer B.Cu) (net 10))
 (segment (start 93.581533 120.836775) (end 94.799535 119.618773) (width 0.2) (layer B.Cu) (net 10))
 (segment (start 93.581533 121.011775) (end 93.581533 120.836775) (width 0.2) (layer B.Cu) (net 10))
 (segment (start 97.349536 114.244774) (end 97.429534 114.164776) (width 0.2) (layer B.Cu) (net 10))
 (segment (start 108.811533 113.592775) (end 101.442543 113.592775) (width 0.2) (layer F.Cu) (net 10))
 (via (at 85.450033 110.511275) (size 0.6) (drill 0.4) (layers F.Cu B.Cu) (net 4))
 (segment (start 85.961533 108.773775) (end 85.961533 109.999775) (width 0.2) (layer B.Cu) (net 4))
 (segment (start 85.961533 109.999775) (end 85.450033 110.511275) (width 0.2) (layer B.Cu) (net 4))
 (segment (start 85.450033 109.901775) (end 85.539033 109.812775) (width 0.2) (layer F.Cu) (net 4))
 (segment (start 85.450033 110.511275) (end 85.450033 109.901775) (width 0.2) (layer F.Cu) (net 4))
 (segment (start 83.964033 109.812775) (end 83.964033 111.717775) (width 0.2) (layer F.Cu) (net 5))
 (segment (start 83.964033 116.797775) (end 83.964033 114.892775) (width 0.2) (layer F.Cu) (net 6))
 (segment (start 86.469533 117.728275) (end 86.469533 118.933775) (width 0.2) (layer F.Cu) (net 7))
 (segment (start 85.539033 116.797775) (end 86.469533 117.728275) (width 0.2) (layer F.Cu) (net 7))
 (segment (start 84.801523 117.835765) (end 84.801523 116.049285) (width 0.2) (layer F.Cu) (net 14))
 (segment (start 85.199533 118.933775) (end 85.199533 118.233775) (width 0.2) (layer F.Cu) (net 14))
 (segment (start 85.199533 118.233775) (end 84.801523 117.835765) (width 0.2) (layer F.Cu) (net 14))
 (segment (start 84.801523 116.049285) (end 85.069033 115.781775) (width 0.2) (layer F.Cu) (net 14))
 (segment (start 86.724533 115.302775) (end 86.724533 114.502775) (width 0.2) (layer F.Cu) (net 14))
 (segment (start 86.245533 115.781775) (end 86.724533 115.302775) (width 0.2) (layer F.Cu) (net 14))
 (segment (start 85.069033 115.781775) (end 86.245533 115.781775) (width 0.2) (layer F.Cu) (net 14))
 (segment (start 86.724533 110.202775) (end 86.724533 110.477775) (width 0.2) (layer F.Cu) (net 14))
 (segment (start 87.249533 111.002775) (end 87.249533 113.702775) (width 0.2) (layer F.Cu) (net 14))
 (segment (start 87.249533 113.702775) (end 86.724533 114.227775) (width 0.2) (layer F.Cu) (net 14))
 (segment (start 86.724533 110.477775) (end 87.249533 111.002775) (width 0.2) (layer F.Cu) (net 14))
 (segment (start 86.724533 114.227775) (end 86.724533 114.502775) (width 0.2) (layer F.Cu) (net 14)))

